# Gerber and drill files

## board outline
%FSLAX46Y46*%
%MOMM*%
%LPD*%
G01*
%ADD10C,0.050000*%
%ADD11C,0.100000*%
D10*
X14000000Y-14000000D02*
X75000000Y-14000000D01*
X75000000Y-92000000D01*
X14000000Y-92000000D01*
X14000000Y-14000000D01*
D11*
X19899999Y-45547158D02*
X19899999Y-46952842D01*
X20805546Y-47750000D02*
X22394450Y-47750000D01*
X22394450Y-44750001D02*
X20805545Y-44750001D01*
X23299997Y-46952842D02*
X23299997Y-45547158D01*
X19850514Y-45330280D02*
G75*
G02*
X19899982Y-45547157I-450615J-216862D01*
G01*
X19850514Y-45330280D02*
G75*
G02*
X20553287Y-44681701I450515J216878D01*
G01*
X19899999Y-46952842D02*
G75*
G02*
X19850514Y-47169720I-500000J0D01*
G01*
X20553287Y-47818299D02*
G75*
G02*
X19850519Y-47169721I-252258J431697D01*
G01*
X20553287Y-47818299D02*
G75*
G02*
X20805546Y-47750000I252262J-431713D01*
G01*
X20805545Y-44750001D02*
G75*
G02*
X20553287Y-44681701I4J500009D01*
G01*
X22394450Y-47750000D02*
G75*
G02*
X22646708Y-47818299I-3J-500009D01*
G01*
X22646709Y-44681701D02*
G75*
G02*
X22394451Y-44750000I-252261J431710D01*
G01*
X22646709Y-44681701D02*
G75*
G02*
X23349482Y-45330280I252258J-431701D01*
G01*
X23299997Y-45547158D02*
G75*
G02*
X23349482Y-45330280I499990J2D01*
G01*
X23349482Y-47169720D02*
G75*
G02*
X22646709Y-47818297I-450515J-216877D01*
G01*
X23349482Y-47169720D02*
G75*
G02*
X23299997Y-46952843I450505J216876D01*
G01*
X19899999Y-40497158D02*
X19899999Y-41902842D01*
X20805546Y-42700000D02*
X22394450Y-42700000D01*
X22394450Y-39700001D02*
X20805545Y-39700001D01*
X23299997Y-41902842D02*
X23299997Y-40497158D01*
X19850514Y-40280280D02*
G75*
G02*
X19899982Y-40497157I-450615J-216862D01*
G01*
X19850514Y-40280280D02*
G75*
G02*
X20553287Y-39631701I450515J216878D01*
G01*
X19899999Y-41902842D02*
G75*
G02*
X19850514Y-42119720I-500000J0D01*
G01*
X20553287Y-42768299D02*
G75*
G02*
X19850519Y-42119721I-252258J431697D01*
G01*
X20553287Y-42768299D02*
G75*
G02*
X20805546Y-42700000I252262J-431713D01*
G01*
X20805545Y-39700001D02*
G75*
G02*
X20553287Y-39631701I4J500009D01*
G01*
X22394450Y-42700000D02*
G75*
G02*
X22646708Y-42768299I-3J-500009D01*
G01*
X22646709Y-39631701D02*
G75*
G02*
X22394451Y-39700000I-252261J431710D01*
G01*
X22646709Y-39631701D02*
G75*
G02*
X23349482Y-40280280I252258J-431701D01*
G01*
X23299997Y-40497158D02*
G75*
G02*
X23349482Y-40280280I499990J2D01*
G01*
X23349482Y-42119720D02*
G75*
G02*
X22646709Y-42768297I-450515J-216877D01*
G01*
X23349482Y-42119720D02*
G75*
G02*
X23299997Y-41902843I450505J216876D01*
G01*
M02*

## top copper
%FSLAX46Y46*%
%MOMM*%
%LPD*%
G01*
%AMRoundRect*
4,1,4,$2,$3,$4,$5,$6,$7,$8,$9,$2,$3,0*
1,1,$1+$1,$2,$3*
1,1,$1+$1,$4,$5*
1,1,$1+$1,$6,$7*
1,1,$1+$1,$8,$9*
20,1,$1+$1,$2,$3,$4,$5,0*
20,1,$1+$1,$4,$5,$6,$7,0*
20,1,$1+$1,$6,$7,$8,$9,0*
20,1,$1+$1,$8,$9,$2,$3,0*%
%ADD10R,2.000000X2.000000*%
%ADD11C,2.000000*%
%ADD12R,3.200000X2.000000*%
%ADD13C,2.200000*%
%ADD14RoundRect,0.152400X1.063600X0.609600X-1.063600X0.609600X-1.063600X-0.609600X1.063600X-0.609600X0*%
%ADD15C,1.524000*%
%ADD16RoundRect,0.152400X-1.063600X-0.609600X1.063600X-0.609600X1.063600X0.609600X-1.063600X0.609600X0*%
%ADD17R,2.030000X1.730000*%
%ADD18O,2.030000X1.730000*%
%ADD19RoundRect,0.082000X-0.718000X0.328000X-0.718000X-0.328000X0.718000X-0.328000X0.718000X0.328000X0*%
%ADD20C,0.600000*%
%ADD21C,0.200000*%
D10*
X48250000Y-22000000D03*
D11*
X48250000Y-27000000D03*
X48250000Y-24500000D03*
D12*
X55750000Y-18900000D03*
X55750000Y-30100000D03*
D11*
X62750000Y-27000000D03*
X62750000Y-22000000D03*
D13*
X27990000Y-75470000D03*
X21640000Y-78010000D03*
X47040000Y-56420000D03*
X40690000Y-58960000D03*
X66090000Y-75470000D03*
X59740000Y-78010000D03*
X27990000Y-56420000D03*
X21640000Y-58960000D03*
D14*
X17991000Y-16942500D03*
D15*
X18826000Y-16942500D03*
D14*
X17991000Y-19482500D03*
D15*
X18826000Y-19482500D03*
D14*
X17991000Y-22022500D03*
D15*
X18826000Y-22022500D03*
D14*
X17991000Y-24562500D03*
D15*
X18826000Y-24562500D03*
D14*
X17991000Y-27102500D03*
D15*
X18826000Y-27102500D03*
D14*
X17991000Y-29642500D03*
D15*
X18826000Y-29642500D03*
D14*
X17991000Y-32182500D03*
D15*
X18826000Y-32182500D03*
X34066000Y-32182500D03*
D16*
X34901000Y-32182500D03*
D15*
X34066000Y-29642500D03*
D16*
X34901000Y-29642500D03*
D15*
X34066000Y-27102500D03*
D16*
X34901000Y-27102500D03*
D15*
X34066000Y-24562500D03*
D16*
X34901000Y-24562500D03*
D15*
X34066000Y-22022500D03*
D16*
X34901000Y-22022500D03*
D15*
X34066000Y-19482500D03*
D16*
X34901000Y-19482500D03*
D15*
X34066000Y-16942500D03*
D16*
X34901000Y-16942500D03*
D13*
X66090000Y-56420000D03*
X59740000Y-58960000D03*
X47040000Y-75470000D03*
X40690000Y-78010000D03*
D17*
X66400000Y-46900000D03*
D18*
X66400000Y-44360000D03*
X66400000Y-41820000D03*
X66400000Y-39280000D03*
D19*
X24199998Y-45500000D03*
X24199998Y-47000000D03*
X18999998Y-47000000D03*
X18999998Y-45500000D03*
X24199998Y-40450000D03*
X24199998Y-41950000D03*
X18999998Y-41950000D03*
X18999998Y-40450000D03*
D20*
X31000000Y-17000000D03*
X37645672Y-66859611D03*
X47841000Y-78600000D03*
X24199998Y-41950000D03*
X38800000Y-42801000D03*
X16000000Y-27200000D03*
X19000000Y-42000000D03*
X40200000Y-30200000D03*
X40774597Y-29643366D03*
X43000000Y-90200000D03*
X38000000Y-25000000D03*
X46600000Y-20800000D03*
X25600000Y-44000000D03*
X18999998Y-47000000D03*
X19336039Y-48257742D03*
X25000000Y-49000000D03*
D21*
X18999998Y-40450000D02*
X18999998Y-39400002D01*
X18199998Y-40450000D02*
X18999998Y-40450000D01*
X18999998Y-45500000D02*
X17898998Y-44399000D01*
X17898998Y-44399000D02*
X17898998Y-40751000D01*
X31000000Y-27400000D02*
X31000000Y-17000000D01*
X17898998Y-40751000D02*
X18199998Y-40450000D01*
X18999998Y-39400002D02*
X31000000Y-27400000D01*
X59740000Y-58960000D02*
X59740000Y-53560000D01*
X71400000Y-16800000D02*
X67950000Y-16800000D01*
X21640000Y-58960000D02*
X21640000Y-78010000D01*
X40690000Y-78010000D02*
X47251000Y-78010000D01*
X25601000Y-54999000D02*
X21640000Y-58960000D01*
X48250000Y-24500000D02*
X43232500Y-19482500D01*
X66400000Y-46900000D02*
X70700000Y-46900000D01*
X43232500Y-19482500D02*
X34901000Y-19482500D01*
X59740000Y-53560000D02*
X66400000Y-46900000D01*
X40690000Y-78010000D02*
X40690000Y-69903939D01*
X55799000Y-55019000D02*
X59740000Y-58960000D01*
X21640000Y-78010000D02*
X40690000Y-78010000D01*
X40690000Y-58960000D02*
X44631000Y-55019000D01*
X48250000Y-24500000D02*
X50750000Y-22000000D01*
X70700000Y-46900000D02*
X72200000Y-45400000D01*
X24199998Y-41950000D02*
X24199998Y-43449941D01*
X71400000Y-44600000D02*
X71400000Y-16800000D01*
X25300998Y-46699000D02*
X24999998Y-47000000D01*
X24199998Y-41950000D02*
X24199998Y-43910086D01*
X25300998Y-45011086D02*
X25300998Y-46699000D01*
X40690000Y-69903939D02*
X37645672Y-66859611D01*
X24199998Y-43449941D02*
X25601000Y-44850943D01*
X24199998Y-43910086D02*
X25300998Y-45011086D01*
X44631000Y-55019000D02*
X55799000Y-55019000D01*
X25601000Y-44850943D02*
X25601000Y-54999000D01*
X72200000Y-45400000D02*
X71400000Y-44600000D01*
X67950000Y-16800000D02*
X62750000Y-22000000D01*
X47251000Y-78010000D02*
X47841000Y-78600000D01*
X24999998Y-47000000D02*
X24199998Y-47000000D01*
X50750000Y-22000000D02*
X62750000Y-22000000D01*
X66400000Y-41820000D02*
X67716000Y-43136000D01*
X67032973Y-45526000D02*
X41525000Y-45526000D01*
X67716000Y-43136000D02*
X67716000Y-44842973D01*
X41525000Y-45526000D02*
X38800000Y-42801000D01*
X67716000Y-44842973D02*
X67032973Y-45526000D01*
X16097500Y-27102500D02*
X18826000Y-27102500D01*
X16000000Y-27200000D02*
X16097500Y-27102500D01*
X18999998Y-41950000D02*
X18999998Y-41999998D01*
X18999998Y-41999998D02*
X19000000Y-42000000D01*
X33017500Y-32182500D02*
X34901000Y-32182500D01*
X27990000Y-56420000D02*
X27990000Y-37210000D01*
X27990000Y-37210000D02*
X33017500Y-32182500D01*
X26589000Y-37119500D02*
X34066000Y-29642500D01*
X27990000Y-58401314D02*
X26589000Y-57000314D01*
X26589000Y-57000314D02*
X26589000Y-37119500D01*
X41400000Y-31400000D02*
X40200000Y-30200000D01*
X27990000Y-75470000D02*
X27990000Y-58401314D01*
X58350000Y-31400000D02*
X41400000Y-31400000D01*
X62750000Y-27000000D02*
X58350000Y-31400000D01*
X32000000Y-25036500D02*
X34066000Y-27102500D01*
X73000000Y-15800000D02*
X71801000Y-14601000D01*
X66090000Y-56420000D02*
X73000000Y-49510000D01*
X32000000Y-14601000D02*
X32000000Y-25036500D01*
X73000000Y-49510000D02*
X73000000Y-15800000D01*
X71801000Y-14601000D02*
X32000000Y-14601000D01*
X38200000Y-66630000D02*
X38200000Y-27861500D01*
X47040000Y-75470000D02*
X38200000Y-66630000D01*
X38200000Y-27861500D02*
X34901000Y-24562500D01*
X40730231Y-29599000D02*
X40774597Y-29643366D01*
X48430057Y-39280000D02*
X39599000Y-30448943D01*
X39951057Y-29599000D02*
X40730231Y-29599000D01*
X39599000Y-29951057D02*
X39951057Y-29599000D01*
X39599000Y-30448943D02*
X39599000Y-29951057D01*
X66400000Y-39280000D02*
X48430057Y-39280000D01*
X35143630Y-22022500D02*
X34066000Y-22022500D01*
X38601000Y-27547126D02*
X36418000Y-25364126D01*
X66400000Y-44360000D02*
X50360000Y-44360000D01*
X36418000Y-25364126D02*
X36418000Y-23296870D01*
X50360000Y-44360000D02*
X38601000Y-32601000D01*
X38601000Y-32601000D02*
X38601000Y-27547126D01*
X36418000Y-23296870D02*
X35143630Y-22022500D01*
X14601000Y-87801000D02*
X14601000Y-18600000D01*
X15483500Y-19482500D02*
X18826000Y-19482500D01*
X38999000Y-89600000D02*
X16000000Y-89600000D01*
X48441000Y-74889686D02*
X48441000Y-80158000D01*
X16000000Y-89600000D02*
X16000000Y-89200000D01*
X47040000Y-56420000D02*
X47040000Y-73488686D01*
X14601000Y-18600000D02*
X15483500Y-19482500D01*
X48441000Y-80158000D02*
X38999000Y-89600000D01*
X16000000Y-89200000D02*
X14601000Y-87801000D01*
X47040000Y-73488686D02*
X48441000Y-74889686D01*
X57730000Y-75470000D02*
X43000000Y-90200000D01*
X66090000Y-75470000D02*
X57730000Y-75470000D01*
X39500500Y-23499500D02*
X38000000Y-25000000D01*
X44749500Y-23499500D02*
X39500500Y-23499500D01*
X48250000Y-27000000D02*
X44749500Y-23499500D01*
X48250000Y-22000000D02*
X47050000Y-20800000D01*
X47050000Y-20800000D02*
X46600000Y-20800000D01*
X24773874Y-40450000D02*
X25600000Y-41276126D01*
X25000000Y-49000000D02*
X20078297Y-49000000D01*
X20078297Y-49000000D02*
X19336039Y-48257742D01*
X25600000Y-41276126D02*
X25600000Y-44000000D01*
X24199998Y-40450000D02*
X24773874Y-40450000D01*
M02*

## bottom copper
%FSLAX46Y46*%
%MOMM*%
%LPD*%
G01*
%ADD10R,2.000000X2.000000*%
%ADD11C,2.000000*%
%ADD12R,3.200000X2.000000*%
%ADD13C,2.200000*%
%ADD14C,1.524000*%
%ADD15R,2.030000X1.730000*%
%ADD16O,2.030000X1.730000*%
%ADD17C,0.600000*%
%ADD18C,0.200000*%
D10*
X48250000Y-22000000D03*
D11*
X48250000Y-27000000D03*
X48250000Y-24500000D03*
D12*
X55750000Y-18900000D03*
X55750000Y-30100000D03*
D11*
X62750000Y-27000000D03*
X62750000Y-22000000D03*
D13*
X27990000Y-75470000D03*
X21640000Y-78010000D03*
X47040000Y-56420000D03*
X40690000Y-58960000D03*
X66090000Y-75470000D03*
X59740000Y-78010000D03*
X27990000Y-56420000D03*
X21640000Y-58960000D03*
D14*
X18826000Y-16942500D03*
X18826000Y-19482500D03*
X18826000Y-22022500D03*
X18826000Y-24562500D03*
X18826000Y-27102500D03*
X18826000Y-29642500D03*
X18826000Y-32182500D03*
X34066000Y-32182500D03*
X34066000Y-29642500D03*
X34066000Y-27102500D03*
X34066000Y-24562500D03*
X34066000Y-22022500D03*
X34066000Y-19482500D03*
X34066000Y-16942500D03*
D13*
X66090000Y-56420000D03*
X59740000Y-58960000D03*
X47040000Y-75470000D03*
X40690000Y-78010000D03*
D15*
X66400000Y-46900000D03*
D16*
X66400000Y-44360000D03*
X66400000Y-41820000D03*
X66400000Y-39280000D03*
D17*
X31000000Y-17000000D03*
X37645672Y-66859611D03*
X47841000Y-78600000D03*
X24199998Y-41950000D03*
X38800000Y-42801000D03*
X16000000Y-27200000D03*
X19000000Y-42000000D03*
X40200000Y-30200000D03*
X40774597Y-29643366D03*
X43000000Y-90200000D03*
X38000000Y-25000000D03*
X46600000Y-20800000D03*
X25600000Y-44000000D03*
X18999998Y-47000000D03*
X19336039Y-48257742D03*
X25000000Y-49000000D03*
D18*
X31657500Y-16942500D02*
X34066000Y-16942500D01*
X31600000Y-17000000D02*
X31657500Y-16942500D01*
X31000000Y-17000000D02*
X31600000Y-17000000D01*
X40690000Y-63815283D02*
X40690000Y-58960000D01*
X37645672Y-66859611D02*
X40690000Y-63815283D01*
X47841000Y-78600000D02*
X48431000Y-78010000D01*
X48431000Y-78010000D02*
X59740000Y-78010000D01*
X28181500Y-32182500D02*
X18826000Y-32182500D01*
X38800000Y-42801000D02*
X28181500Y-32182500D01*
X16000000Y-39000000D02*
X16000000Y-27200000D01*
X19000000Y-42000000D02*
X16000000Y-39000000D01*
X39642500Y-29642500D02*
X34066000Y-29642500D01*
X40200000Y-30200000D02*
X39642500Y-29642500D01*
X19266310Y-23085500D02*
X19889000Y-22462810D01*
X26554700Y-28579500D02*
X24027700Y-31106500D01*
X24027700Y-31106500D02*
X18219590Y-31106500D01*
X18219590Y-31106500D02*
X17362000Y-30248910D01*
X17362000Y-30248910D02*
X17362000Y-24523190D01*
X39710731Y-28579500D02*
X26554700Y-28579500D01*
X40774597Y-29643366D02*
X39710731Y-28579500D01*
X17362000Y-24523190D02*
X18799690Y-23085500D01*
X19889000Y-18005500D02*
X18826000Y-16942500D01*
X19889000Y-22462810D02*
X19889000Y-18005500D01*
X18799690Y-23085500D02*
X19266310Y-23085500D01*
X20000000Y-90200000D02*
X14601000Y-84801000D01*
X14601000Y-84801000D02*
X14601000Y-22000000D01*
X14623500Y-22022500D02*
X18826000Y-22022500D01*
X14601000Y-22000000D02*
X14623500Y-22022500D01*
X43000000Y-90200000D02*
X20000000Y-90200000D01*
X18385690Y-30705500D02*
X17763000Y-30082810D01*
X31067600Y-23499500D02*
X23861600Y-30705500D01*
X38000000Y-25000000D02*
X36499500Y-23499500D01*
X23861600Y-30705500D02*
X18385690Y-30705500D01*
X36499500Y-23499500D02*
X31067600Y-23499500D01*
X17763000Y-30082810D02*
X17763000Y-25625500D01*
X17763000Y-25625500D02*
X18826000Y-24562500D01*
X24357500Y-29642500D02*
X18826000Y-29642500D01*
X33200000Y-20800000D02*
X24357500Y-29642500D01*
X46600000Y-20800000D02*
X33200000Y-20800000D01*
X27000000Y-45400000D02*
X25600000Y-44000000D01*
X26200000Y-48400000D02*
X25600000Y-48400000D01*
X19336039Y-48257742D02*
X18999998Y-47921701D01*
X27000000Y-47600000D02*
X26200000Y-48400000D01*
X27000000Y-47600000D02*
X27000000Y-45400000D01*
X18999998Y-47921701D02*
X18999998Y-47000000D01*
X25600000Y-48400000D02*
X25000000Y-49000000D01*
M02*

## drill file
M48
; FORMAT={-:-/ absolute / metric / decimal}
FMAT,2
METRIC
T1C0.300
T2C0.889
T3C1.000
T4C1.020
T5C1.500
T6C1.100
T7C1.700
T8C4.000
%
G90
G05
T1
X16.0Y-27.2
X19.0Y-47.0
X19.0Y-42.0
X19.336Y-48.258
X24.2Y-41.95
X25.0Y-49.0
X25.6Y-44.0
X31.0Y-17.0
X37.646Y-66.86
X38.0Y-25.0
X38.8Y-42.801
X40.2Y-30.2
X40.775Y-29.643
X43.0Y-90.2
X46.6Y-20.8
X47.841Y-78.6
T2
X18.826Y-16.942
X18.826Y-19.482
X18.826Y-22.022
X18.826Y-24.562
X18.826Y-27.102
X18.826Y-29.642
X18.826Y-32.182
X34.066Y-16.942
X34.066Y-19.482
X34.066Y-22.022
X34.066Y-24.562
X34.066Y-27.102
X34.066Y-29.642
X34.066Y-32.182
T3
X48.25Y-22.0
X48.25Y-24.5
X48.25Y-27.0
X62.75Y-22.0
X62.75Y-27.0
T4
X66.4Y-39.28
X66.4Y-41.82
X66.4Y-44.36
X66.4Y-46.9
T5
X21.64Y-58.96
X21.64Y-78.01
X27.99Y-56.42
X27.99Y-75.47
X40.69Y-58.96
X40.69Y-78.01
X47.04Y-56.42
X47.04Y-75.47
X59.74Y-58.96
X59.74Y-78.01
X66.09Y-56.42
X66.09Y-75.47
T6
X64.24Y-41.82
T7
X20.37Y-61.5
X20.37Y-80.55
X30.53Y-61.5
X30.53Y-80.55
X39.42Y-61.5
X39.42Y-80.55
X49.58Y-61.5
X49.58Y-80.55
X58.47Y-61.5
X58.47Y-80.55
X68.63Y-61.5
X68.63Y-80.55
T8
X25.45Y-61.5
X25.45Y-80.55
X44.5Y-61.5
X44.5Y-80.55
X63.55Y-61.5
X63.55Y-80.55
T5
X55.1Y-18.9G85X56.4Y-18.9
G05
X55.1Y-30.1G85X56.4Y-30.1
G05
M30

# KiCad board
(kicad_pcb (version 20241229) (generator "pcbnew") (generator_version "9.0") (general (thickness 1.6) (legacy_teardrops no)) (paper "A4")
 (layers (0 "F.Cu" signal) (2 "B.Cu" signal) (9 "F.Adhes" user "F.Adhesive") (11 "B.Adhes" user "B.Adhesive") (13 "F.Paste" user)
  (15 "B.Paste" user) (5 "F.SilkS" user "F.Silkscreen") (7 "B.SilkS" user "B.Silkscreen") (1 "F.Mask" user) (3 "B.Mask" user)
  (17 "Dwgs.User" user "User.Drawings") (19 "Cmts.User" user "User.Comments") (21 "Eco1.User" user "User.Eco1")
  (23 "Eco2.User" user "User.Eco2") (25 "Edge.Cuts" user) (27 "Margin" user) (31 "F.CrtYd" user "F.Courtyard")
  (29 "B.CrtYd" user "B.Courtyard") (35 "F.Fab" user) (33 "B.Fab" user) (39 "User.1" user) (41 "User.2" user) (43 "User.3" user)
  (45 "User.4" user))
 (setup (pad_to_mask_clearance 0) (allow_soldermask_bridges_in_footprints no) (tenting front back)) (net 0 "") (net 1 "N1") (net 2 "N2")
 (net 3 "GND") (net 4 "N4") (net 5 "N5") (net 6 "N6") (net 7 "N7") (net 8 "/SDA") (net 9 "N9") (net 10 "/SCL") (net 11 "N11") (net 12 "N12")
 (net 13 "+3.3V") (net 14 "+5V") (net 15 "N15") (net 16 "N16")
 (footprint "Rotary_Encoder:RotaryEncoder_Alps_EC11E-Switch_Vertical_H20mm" (layer "F.Cu") (at 48.25 22)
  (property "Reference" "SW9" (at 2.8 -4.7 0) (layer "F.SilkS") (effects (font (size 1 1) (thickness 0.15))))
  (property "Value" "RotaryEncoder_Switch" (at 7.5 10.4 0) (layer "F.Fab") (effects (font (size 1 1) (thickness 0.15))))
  (pad "A" thru_hole rect (at 0 0) (size 2 2) (drill 1) (layers "*.Cu" "*.Mask") (remove_unused_layers no) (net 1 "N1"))
  (pad "B" thru_hole circle (at 0 5) (size 2 2) (drill 1) (layers "*.Cu" "*.Mask") (remove_unused_layers no) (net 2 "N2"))
  (pad "C" thru_hole circle (at 0 2.5) (size 2 2) (drill 1) (layers "*.Cu" "*.Mask") (remove_unused_layers no) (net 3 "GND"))
  (pad "MP" thru_hole rect (at 7.5 -3.1) (size 3.2 2) (drill oval 2.8 1.5) (layers "*.Cu" "*.Mask") (remove_unused_layers no))
  (pad "MP" thru_hole rect (at 7.5 8.1) (size 3.2 2) (drill oval 2.8 1.5) (layers "*.Cu" "*.Mask") (remove_unused_layers no))
  (pad "S1" thru_hole circle (at 14.5 5) (size 2 2) (drill 1) (layers "*.Cu" "*.Mask") (remove_unused_layers no) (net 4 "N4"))
  (pad "S2" thru_hole circle (at 14.5 0) (size 2 2) (drill 1) (layers "*.Cu" "*.Mask") (remove_unused_layers no) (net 3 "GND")))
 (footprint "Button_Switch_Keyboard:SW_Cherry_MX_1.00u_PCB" (layer "F.Cu") (at 27.99 75.47)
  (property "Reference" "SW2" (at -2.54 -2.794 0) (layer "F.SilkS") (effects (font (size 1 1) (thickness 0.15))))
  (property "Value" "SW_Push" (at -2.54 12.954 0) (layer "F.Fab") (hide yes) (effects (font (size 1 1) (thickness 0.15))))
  (pad "" np_thru_hole circle (at -7.62 5.08) (size 1.7 1.7) (drill 1.7) (layers "*.Cu" "*.Mask"))
  (pad "" np_thru_hole circle (at -2.54 5.08) (size 4 4) (drill 4) (layers "*.Cu" "*.Mask"))
  (pad "" np_thru_hole circle (at 2.54 5.08) (size 1.7 1.7) (drill 1.7) (layers "*.Cu" "*.Mask"))
  (pad "1" thru_hole circle (at 0 0) (size 2.2 2.2) (drill 1.5) (layers "*.Cu" "*.Mask") (remove_unused_layers no) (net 4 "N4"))
  (pad "2" thru_hole circle (at -6.35 2.54) (size 2.2 2.2) (drill 1.5) (layers "*.Cu" "*.Mask") (remove_unused_layers no) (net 3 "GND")))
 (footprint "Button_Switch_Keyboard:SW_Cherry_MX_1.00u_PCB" (layer "F.Cu") (at 47.04 56.42)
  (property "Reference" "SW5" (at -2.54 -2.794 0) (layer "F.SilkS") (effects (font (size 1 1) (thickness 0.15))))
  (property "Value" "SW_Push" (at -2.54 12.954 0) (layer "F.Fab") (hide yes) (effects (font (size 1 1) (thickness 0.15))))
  (pad "" np_thru_hole circle (at -7.62 5.08) (size 1.7 1.7) (drill 1.7) (layers "*.Cu" "*.Mask"))
  (pad "" np_thru_hole circle (at -2.54 5.08) (size 4 4) (drill 4) (layers "*.Cu" "*.Mask"))
  (pad "" np_thru_hole circle (at 2.54 5.08) (size 1.7 1.7) (drill 1.7) (layers "*.Cu" "*.Mask"))
  (pad "1" thru_hole circle (at 0 0) (size 2.2 2.2) (drill 1.5) (layers "*.Cu" "*.Mask") (remove_unused_layers no) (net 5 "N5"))
  (pad "2" thru_hole circle (at -6.35 2.54) (size 2.2 2.2) (drill 1.5) (layers "*.Cu" "*.Mask") (remove_unused_layers no) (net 3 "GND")))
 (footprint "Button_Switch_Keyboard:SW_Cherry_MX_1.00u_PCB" (layer "F.Cu") (at 66.09 75.47)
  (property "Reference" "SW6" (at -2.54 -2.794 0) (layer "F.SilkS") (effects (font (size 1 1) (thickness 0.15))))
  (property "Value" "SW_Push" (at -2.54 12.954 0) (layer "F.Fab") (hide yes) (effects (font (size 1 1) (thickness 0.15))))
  (pad "" np_thru_hole circle (at -7.62 5.08) (size 1.7 1.7) (drill 1.7) (layers "*.Cu" "*.Mask"))
  (pad "" np_thru_hole circle (at -2.54 5.08) (size 4 4) (drill 4) (layers "*.Cu" "*.Mask"))
  (pad "" np_thru_hole circle (at 2.54 5.08) (size 1.7 1.7) (drill 1.7) (layers "*.Cu" "*.Mask"))
  (pad "1" thru_hole circle (at 0 0) (size 2.2 2.2) (drill 1.5) (layers "*.Cu" "*.Mask") (remove_unused_layers no) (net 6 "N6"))
  (pad "2" thru_hole circle (at -6.35 2.54) (size 2.2 2.2) (drill 1.5) (layers "*.Cu" "*.Mask") (remove_unused_layers no) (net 3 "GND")))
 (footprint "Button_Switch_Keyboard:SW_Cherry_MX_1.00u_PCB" (layer "F.Cu") (at 27.99 56.42)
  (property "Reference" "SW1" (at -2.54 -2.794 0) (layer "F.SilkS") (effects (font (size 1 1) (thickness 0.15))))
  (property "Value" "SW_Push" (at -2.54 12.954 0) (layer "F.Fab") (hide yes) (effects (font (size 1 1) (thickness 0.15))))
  (pad "" np_thru_hole circle (at -7.62 5.08) (size 1.7 1.7) (drill 1.7) (layers "*.Cu" "*.Mask"))
  (pad "" np_thru_hole circle (at -2.54 5.08) (size 4 4) (drill 4) (layers "*.Cu" "*.Mask"))
  (pad "" np_thru_hole circle (at 2.54 5.08) (size 1.7 1.7) (drill 1.7) (layers "*.Cu" "*.Mask"))
  (pad "1" thru_hole circle (at 0 0) (size 2.2 2.2) (drill 1.5) (layers "*.Cu" "*.Mask") (remove_unused_layers no) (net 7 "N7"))
  (pad "2" thru_hole circle (at -6.35 2.54) (size 2.2 2.2) (drill 1.5) (layers "*.Cu" "*.Mask") (remove_unused_layers no) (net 3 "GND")))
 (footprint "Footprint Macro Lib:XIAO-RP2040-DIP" (layer "F.Cu") (at 26.446 24.5625)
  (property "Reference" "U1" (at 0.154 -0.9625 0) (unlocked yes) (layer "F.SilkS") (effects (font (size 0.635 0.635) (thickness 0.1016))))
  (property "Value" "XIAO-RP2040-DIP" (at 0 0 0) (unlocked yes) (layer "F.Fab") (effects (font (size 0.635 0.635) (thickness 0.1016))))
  (pad "1" smd roundrect (at -8.455 -7.62 180) (size 2.432 1.524) (layers "F.Cu" "F.Mask") (roundrect_rratio 0.1) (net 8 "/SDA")
   (thermal_bridge_angle 45))
  (pad "1" thru_hole circle (at -7.62 -7.62 180) (size 1.524 1.524) (drill 0.889) (layers "*.Cu" "*.Mask") (remove_unused_layers no)
   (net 8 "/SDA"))
  (pad "2" smd roundrect (at -8.455 -5.08 180) (size 2.432 1.524) (layers "F.Cu" "F.Mask") (roundrect_rratio 0.1) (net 5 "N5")
   (thermal_bridge_angle 45))
  (pad "2" thru_hole circle (at -7.62 -5.08 180) (size 1.524 1.524) (drill 0.889) (layers "*.Cu" "*.Mask") (remove_unused_layers no)
   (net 5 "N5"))
  (pad "3" smd roundrect (at -8.455 -2.54 180) (size 2.432 1.524) (layers "F.Cu" "F.Mask") (roundrect_rratio 0.1) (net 6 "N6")
   (thermal_bridge_angle 45))
  (pad "3" thru_hole circle (at -7.62 -2.54 180) (size 1.524 1.524) (drill 0.889) (layers "*.Cu" "*.Mask") (remove_unused_layers no)
   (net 6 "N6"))
  (pad "4" smd roundrect (at -8.455 0 180) (size 2.432 1.524) (layers "F.Cu" "F.Mask") (roundrect_rratio 0.1) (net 2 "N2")
   (thermal_bridge_angle 45))
  (pad "4" thru_hole circle (at -7.62 0 180) (size 1.524 1.524) (drill 0.889) (layers "*.Cu" "*.Mask") (remove_unused_layers no)
   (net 2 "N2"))
  (pad "5" smd roundrect (at -8.455 2.54 180) (size 2.432 1.524) (layers "F.Cu" "F.Mask") (roundrect_rratio 0.1) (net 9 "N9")
   (thermal_bridge_angle 45))
  (pad "5" thru_hole circle (at -7.62 2.54 180) (size 1.524 1.524) (drill 0.889) (layers "*.Cu" "*.Mask") (remove_unused_layers no)
   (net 9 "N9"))
  (pad "6" smd roundrect (at -8.455 5.08 180) (size 2.432 1.524) (layers "F.Cu" "F.Mask") (roundrect_rratio 0.1) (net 1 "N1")
   (thermal_bridge_angle 45))
  (pad "6" thru_hole circle (at -7.62 5.08 180) (size 1.524 1.524) (drill 0.889) (layers "*.Cu" "*.Mask") (remove_unused_layers no)
   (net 1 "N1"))
  (pad "7" smd roundrect (at -8.455 7.62 180) (size 2.432 1.524) (layers "F.Cu" "F.Mask") (roundrect_rratio 0.1) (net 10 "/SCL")
   (thermal_bridge_angle 45))
  (pad "7" thru_hole circle (at -7.62 7.62 180) (size 1.524 1.524) (drill 0.889) (layers "*.Cu" "*.Mask") (remove_unused_layers no)
   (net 10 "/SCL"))
  (pad "8" thru_hole circle (at 7.62 7.62) (size 1.524 1.524) (drill 0.889) (layers "*.Cu" "*.Mask") (remove_unused_layers no) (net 7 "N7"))
  (pad "8" smd roundrect (at 8.455 7.62) (size 2.432 1.524) (layers "F.Cu" "F.Mask") (roundrect_rratio 0.1) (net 7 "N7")
   (thermal_bridge_angle 45))
  (pad "9" thru_hole circle (at 7.62 5.08) (size 1.524 1.524) (drill 0.889) (layers "*.Cu" "*.Mask") (remove_unused_layers no) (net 4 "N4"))
  (pad "9" smd roundrect (at 8.455 5.08) (size 2.432 1.524) (layers "F.Cu" "F.Mask") (roundrect_rratio 0.1) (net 4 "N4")
   (thermal_bridge_angle 45))
  (pad "10" thru_hole circle (at 7.62 2.54) (size 1.524 1.524) (drill 0.889) (layers "*.Cu" "*.Mask") (remove_unused_layers no)
   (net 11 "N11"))
  (pad "10" smd roundrect (at 8.455 2.54) (size 2.432 1.524) (layers "F.Cu" "F.Mask") (roundrect_rratio 0.1) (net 11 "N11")
   (thermal_bridge_angle 45))
  (pad "11" thru_hole circle (at 7.62 0) (size 1.524 1.524) (drill 0.889) (layers "*.Cu" "*.Mask") (remove_unused_layers no) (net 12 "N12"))
  (pad "11" smd roundrect (at 8.455 0) (size 2.432 1.524) (layers "F.Cu" "F.Mask") (roundrect_rratio 0.1) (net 12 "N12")
   (thermal_bridge_angle 45))
  (pad "12" thru_hole circle (at 7.62 -2.54) (size 1.524 1.524) (drill 0.889) (layers "*.Cu" "*.Mask") (remove_unused_layers no)
   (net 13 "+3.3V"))
  (pad "12" smd roundrect (at 8.455 -2.54) (size 2.432 1.524) (layers "F.Cu" "F.Mask") (roundrect_rratio 0.1) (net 13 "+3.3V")
   (thermal_bridge_angle 45))
  (pad "13" thru_hole circle (at 7.62 -5.08) (size 1.524 1.524) (drill 0.889) (layers "*.Cu" "*.Mask") (remove_unused_layers no)
   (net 3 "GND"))
  (pad "13" smd roundrect (at 8.455 -5.08) (size 2.432 1.524) (layers "F.Cu" "F.Mask") (roundrect_rratio 0.1) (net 3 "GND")
   (thermal_bridge_angle 45))
  (pad "14" thru_hole circle (at 7.62 -7.62) (size 1.524 1.524) (drill 0.889) (layers "*.Cu" "*.Mask") (remove_unused_layers no)
   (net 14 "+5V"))
  (pad "14" smd roundrect (at 8.455 -7.62) (size 2.432 1.524) (layers "F.Cu" "F.Mask") (roundrect_rratio 0.1) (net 14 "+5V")
   (thermal_bridge_angle 45)))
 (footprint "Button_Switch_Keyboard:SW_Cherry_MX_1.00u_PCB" (layer "F.Cu") (at 66.09 56.42)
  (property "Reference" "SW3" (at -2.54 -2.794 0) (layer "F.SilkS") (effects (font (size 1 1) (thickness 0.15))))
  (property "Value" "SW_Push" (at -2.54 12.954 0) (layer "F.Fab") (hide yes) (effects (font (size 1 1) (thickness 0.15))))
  (pad "" np_thru_hole circle (at -7.62 5.08) (size 1.7 1.7) (drill 1.7) (layers "*.Cu" "*.Mask"))
  (pad "" np_thru_hole circle (at -2.54 5.08) (size 4 4) (drill 4) (layers "*.Cu" "*.Mask"))
  (pad "" np_thru_hole circle (at 2.54 5.08) (size 1.7 1.7) (drill 1.7) (layers "*.Cu" "*.Mask"))
  (pad "1" thru_hole circle (at 0 0) (size 2.2 2.2) (drill 1.5) (layers "*.Cu" "*.Mask") (remove_unused_layers no) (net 11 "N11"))
  (pad "2" thru_hole circle (at -6.35 2.54) (size 2.2 2.2) (drill 1.5) (layers "*.Cu" "*.Mask") (remove_unused_layers no) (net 3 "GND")))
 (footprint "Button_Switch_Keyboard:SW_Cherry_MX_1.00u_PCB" (layer "F.Cu") (at 47.04 75.47)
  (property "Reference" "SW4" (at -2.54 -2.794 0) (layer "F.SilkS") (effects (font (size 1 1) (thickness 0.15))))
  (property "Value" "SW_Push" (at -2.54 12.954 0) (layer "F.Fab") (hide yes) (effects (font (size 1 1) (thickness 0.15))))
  (pad "" np_thru_hole circle (at -7.62 5.08) (size 1.7 1.7) (drill 1.7) (layers "*.Cu" "*.Mask"))
  (pad "" np_thru_hole circle (at -2.54 5.08) (size 4 4) (drill 4) (layers "*.Cu" "*.Mask"))
  (pad "" np_thru_hole circle (at 2.54 5.08) (size 1.7 1.7) (drill 1.7) (layers "*.Cu" "*.Mask"))
  (pad "1" thru_hole circle (at 0 0) (size 2.2 2.2) (drill 1.5) (layers "*.Cu" "*.Mask") (remove_unused_layers no) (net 12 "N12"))
  (pad "2" thru_hole circle (at -6.35 2.54) (size 2.2 2.2) (drill 1.5) (layers "*.Cu" "*.Mask") (remove_unused_layers no) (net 3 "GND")))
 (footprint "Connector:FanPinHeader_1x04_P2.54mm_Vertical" (layer "F.Cu") (at 66.4 46.9 90)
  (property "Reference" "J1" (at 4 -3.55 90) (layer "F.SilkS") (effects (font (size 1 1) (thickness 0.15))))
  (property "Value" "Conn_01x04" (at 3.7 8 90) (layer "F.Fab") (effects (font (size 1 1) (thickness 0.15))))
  (pad "" np_thru_hole circle (at 5.08 -2.16 180) (size 1.1 1.1) (drill 1.1) (layers "*.Cu" "*.Mask"))
  (pad "1" thru_hole rect (at 0 0 180) (size 2.03 1.73) (drill 1.02) (layers "*.Cu" "*.Mask") (remove_unused_layers no) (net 3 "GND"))
  (pad "2" thru_hole oval (at 2.54 0 180) (size 2.03 1.73) (drill 1.02) (layers "*.Cu" "*.Mask") (remove_unused_layers no) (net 13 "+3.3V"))
  (pad "3" thru_hole oval (at 5.08 0 180) (size 2.03 1.73) (drill 1.02) (layers "*.Cu" "*.Mask") (remove_unused_layers no) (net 10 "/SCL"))
  (pad "4" thru_hole oval (at 7.62 0 180) (size 2.03 1.73) (drill 1.02) (layers "*.Cu" "*.Mask") (remove_unused_layers no) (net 8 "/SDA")))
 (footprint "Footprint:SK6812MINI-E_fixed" (layer "B.Cu") (at 21.599999 46.352842 180)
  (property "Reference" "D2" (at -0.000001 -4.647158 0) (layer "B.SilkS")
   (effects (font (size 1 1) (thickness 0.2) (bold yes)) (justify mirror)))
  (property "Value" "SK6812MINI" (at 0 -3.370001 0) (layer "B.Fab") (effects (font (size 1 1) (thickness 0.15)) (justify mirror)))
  (fp_line (start 1.7 0.805684) (end 1.7 -0.6) (stroke (width 0.1) (type solid)) (layer "Edge.Cuts"))
  (fp_line (start 0.794453 -1.397158) (end -0.794451 -1.397158) (stroke (width 0.1) (type solid)) (layer "Edge.Cuts"))
  (fp_line (start -0.794451 1.602841) (end 0.794454 1.602841) (stroke (width 0.1) (type solid)) (layer "Edge.Cuts"))
  (fp_line (start -1.699998 -0.6) (end -1.699998 0.805684) (stroke (width 0.1) (type solid)) (layer "Edge.Cuts"))
  (fp_arc (start 1.749485 1.022562) (mid 1.712532 0.91691) (end 1.7 0.805685) (stroke (width 0.1) (type solid)) (layer "Edge.Cuts"))
  (fp_arc (start 1.749485 1.022562) (mid 1.638072 1.606877) (end 1.046712 1.67114) (stroke (width 0.1) (type solid)) (layer "Edge.Cuts"))
  (fp_arc (start 1.7 -0.6) (mid 1.712528 -0.711226) (end 1.749485 -0.816878) (stroke (width 0.1) (type solid)) (layer "Edge.Cuts"))
  (fp_arc (start 1.046712 -1.465457) (mid 1.638073 -1.401193) (end 1.749485 -0.816877) (stroke (width 0.1) (type solid)) (layer "Edge.Cuts"))
  (fp_arc (start 1.046712 -1.465457) (mid 0.925124 -1.414535) (end 0.794453 -1.397158) (stroke (width 0.1) (type solid)) (layer "Edge.Cuts"))
  (fp_arc (start 0.794454 1.602841) (mid 0.925124 1.620218) (end 1.046712 1.67114) (stroke (width 0.1) (type solid)) (layer "Edge.Cuts"))
  (fp_arc (start -0.794451 -1.397158) (mid -0.925121 -1.414535) (end -1.046709 -1.465457) (stroke (width 0.1) (type solid))
   (layer "Edge.Cuts"))
  (fp_arc (start -1.04671 1.671141) (mid -0.925122 1.620219) (end -0.794452 1.602842) (stroke (width 0.1) (type solid)) (layer "Edge.Cuts"))
  (fp_arc (start -1.04671 1.671141) (mid -1.63807 1.606877) (end -1.749483 1.022562) (stroke (width 0.1) (type solid)) (layer "Edge.Cuts"))
  (fp_arc (start -1.699998 0.805684) (mid -1.712526 0.91691) (end -1.749483 1.022562) (stroke (width 0.1) (type solid)) (layer "Edge.Cuts"))
  (fp_arc (start -1.749483 -0.816878) (mid -1.638069 -1.401192) (end -1.04671 -1.465455) (stroke (width 0.1) (type solid))
   (layer "Edge.Cuts"))
  (fp_arc (start -1.749483 -0.816878) (mid -1.712526 -0.711226) (end -1.699998 -0.600001) (stroke (width 0.1) (type solid))
   (layer "Edge.Cuts"))
  (pad "1" smd roundrect (at -2.599999 0.852842 270) (size 0.82 1.6) (layers "F.Cu" "F.Mask" "F.Paste") (roundrect_rratio 0.1)
   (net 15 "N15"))
  (pad "2" smd roundrect (at -2.599999 -0.647158 270) (size 0.82 1.6) (layers "F.Cu" "F.Mask" "F.Paste") (roundrect_rratio 0.1)
   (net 3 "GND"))
  (pad "3" smd roundrect (at 2.600001 -0.647158 270) (size 0.82 1.6) (layers "F.Cu" "F.Mask" "F.Paste") (roundrect_rratio 0.1)
   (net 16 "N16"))
  (pad "4" smd roundrect (at 2.600001 0.852842 270) (size 0.82 1.6) (layers "F.Cu" "F.Mask" "F.Paste") (roundrect_rratio 0.1) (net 14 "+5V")))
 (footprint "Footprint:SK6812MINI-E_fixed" (layer "B.Cu") (at 21.599999 41.302842 180)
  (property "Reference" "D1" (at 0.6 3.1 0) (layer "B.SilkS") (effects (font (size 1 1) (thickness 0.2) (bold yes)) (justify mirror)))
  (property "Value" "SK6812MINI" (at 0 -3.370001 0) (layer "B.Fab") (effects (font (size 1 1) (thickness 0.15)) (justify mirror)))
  (fp_line (start 1.7 0.805684) (end 1.7 -0.6) (stroke (width 0.1) (type solid)) (layer "Edge.Cuts"))
  (fp_line (start 0.794453 -1.397158) (end -0.794451 -1.397158) (stroke (width 0.1) (type solid)) (layer "Edge.Cuts"))
  (fp_line (start -0.794451 1.602841) (end 0.794454 1.602841) (stroke (width 0.1) (type solid)) (layer "Edge.Cuts"))
  (fp_line (start -1.699998 -0.6) (end -1.699998 0.805684) (stroke (width 0.1) (type solid)) (layer "Edge.Cuts"))
  (fp_arc (start 1.749485 1.022562) (mid 1.712532 0.91691) (end 1.7 0.805685) (stroke (width 0.1) (type solid)) (layer "Edge.Cuts"))
  (fp_arc (start 1.749485 1.022562) (mid 1.638072 1.606877) (end 1.046712 1.67114) (stroke (width 0.1) (type solid)) (layer "Edge.Cuts"))
  (fp_arc (start 1.7 -0.6) (mid 1.712528 -0.711226) (end 1.749485 -0.816878) (stroke (width 0.1) (type solid)) (layer "Edge.Cuts"))
  (fp_arc (start 1.046712 -1.465457) (mid 1.638073 -1.401193) (end 1.749485 -0.816877) (stroke (width 0.1) (type solid)) (layer "Edge.Cuts"))
  (fp_arc (start 1.046712 -1.465457) (mid 0.925124 -1.414535) (end 0.794453 -1.397158) (stroke (width 0.1) (type solid)) (layer "Edge.Cuts"))
  (fp_arc (start 0.794454 1.602841) (mid 0.925124 1.620218) (end 1.046712 1.67114) (stroke (width 0.1) (type solid)) (layer "Edge.Cuts"))
  (fp_arc (start -0.794451 -1.397158) (mid -0.925121 -1.414535) (end -1.046709 -1.465457) (stroke (width 0.1) (type solid))
   (layer "Edge.Cuts"))
  (fp_arc (start -1.04671 1.671141) (mid -0.925122 1.620219) (end -0.794452 1.602842) (stroke (width 0.1) (type solid)) (layer "Edge.Cuts"))
  (fp_arc (start -1.04671 1.671141) (mid -1.63807 1.606877) (end -1.749483 1.022562) (stroke (width 0.1) (type solid)) (layer "Edge.Cuts"))
  (fp_arc (start -1.699998 0.805684) (mid -1.712526 0.91691) (end -1.749483 1.022562) (stroke (width 0.1) (type solid)) (layer "Edge.Cuts"))
  (fp_arc (start -1.749483 -0.816878) (mid -1.638069 -1.401192) (end -1.04671 -1.465455) (stroke (width 0.1) (type solid))
   (layer "Edge.Cuts"))
  (fp_arc (start -1.749483 -0.816878) (mid -1.712526 -0.711226) (end -1.699998 -0.600001) (stroke (width 0.1) (type solid))
   (layer "Edge.Cuts"))
  (pad "1" smd roundrect (at -2.599999 0.852842 270) (size 0.82 1.6) (layers "F.Cu" "F.Mask" "F.Paste") (roundrect_rratio 0.1)
   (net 16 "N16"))
  (pad "2" smd roundrect (at -2.599999 -0.647158 270) (size 0.82 1.6) (layers "F.Cu" "F.Mask" "F.Paste") (roundrect_rratio 0.1)
   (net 3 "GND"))
  (pad "3" smd roundrect (at 2.600001 -0.647158 270) (size 0.82 1.6) (layers "F.Cu" "F.Mask" "F.Paste") (roundrect_rratio 0.1) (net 9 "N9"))
  (pad "4" smd roundrect (at 2.600001 0.852842 270) (size 0.82 1.6) (layers "F.Cu" "F.Mask" "F.Paste") (roundrect_rratio 0.1) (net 14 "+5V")))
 (gr_rect (start 14 14) (end 75 92) (stroke (width 0.05) (type solid)) (fill no) (layer "Edge.Cuts"))
 (segment (start 18.999998 40.45) (end 18.999998 39.400002) (width 0.2) (layer "F.Cu") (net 14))
 (segment (start 18.199998 40.45) (end 18.999998 40.45) (width 0.2) (layer "F.Cu") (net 14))
 (segment (start 18.999998 45.5) (end 17.898998 44.399) (width 0.2) (layer "F.Cu") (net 14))
 (segment (start 17.898998 44.399) (end 17.898998 40.751) (width 0.2) (layer "F.Cu") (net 14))
 (segment (start 31 27.4) (end 31 17) (width 0.2) (layer "F.Cu") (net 14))
 (segment (start 17.898998 40.751) (end 18.199998 40.45) (width 0.2) (layer "F.Cu") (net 14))
 (segment (start 18.999998 39.400002) (end 31 27.4) (width 0.2) (layer "F.Cu") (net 14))
 (via (at 31 17) (size 0.6) (drill 0.3) (layers "F.Cu" "B.Cu") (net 14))
 (segment (start 31.6575 16.9425) (end 34.066 16.9425) (width 0.2) (layer "B.Cu") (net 14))
 (segment (start 31.6 17) (end 31.6575 16.9425) (width 0.2) (layer "B.Cu") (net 14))
 (segment (start 31 17) (end 31.6 17) (width 0.2) (layer "B.Cu") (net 14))
 (segment (start 59.74 58.96) (end 59.74 53.56) (width 0.2) (layer "F.Cu") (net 3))
 (segment (start 71.4 16.8) (end 67.95 16.8) (width 0.2) (layer "F.Cu") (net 3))
 (segment (start 21.64 58.96) (end 21.64 78.01) (width 0.2) (layer "F.Cu") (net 3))
 (segment (start 40.69 78.01) (end 47.251 78.01) (width 0.2) (layer "F.Cu") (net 3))
 (segment (start 25.601 54.999) (end 21.64 58.96) (width 0.2) (layer "F.Cu") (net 3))
 (segment (start 48.25 24.5) (end 43.2325 19.4825) (width 0.2) (layer "F.Cu") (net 3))
 (segment (start 66.4 46.9) (end 70.7 46.9) (width 0.2) (layer "F.Cu") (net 3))
 (segment (start 43.2325 19.4825) (end 34.901 19.4825) (width 0.2) (layer "F.Cu") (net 3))
 (segment (start 59.74 53.56) (end 66.4 46.9) (width 0.2) (layer "F.Cu") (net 3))
 (segment (start 40.69 78.01) (end 40.69 69.903939) (width 0.2) (layer "F.Cu") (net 3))
 (segment (start 55.799 55.019) (end 59.74 58.96) (width 0.2) (layer "F.Cu") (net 3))
 (segment (start 21.64 78.01) (end 40.69 78.01) (width 0.2) (layer "F.Cu") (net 3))
 (segment (start 40.69 58.96) (end 44.631 55.019) (width 0.2) (layer "F.Cu") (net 3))
 (segment (start 48.25 24.5) (end 50.75 22) (width 0.2) (layer "F.Cu") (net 3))
 (segment (start 70.7 46.9) (end 72.2 45.4) (width 0.2) (layer "F.Cu") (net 3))
 (segment (start 24.199998 41.95) (end 24.199998 43.449941) (width 0.2) (layer "F.Cu") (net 3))
 (segment (start 71.4 44.6) (end 71.4 16.8) (width 0.2) (layer "F.Cu") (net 3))
 (segment (start 25.300998 46.699) (end 24.999998 47) (width 0.2) (layer "F.Cu") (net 3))
 (segment (start 24.199998 41.95) (end 24.199998 43.910086) (width 0.2) (layer "F.Cu") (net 3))
 (segment (start 25.300998 45.011086) (end 25.300998 46.699) (width 0.2) (layer "F.Cu") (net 3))
 (segment (start 40.69 69.903939) (end 37.645672 66.859611) (width 0.2) (layer "F.Cu") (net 3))
 (segment (start 24.199998 43.449941) (end 25.601 44.850943) (width 0.2) (layer "F.Cu") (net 3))
 (segment (start 24.199998 43.910086) (end 25.300998 45.011086) (width 0.2) (layer "F.Cu") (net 3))
 (segment (start 44.631 55.019) (end 55.799 55.019) (width 0.2) (layer "F.Cu") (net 3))
 (segment (start 25.601 44.850943) (end 25.601 54.999) (width 0.2) (layer "F.Cu") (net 3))
 (segment (start 72.2 45.4) (end 71.4 44.6) (width 0.2) (layer "F.Cu") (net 3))
 (segment (start 67.95 16.8) (end 62.75 22) (width 0.2) (layer "F.Cu") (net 3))
 (segment (start 47.251 78.01) (end 47.841 78.6) (width 0.2) (layer "F.Cu") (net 3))
 (segment (start 24.999998 47) (end 24.199998 47) (width 0.2) (layer "F.Cu") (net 3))
 (segment (start 50.75 22) (end 62.75 22) (width 0.2) (layer "F.Cu") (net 3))
 (via (at 37.645672 66.859611) (size 0.6) (drill 0.3) (layers "F.Cu" "B.Cu") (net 3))
 (via (at 47.841 78.6) (size 0.6) (drill 0.3) (layers "F.Cu" "B.Cu") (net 3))
 (via (at 24.199998 41.95) (size 0.6) (drill 0.3) (layers "F.Cu" "B.Cu") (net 3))
 (segment (start 40.69 63.815283) (end 40.69 58.96) (width 0.2) (layer "B.Cu") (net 3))
 (segment (start 37.645672 66.859611) (end 40.69 63.815283) (width 0.2) (layer "B.Cu") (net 3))
 (segment (start 47.841 78.6) (end 48.431 78.01) (width 0.2) (layer "B.Cu") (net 3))
 (segment (start 48.431 78.01) (end 59.74 78.01) (width 0.2) (layer "B.Cu") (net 3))
 (segment (start 66.4 41.82) (end 67.716 43.136) (width 0.2) (layer "F.Cu") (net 10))
 (segment (start 67.032973 45.526) (end 41.525 45.526) (width 0.2) (layer "F.Cu") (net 10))
 (segment (start 67.716 43.136) (end 67.716 44.842973) (width 0.2) (layer "F.Cu") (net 10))
 (segment (start 41.525 45.526) (end 38.8 42.801) (width 0.2) (layer "F.Cu") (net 10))
 (segment (start 67.716 44.842973) (end 67.032973 45.526) (width 0.2) (layer "F.Cu") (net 10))
 (via (at 38.8 42.801) (size 0.6) (drill 0.3) (layers "F.Cu" "B.Cu") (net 10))
 (segment (start 28.1815 32.1825) (end 18.826 32.1825) (width 0.2) (layer "B.Cu") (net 10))
 (segment (start 38.8 42.801) (end 28.1815 32.1825) (width 0.2) (layer "B.Cu") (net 10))
 (segment (start 16.0975 27.1025) (end 18.826 27.1025) (width 0.2) (layer "F.Cu") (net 9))
 (segment (start 16 27.2) (end 16.0975 27.1025) (width 0.2) (layer "F.Cu") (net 9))
 (segment (start 18.999998 41.95) (end 18.999998 41.999998) (width 0.2) (layer "F.Cu") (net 9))
 (segment (start 18.999998 41.999998) (end 19 42) (width 0.2) (layer "F.Cu") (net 9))
 (via (at 16 27.2) (size 0.6) (drill 0.3) (layers "F.Cu" "B.Cu") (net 9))
 (via (at 19 42) (size 0.6) (drill 0.3) (layers "F.Cu" "B.Cu") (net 9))
 (segment (start 16 39) (end 16 27.2) (width 0.2) (layer "B.Cu") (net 9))
 (segment (start 19 42) (end 16 39) (width 0.2) (layer "B.Cu") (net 9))
 (segment (start 33.0175 32.1825) (end 34.901 32.1825) (width 0.2) (layer "F.Cu") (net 7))
 (segment (start 27.99 56.42) (end 27.99 37.21) (width 0.2) (layer "F.Cu") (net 7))
 (segment (start 27.99 37.21) (end 33.0175 32.1825) (width 0.2) (layer "F.Cu") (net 7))
 (segment (start 26.589 37.1195) (end 34.066 29.6425) (width 0.2) (layer "F.Cu") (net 4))
 (segment (start 27.99 58.401314) (end 26.589 57.000314) (width 0.2) (layer "F.Cu") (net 4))
 (segment (start 26.589 57.000314) (end 26.589 37.1195) (width 0.2) (layer "F.Cu") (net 4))
 (segment (start 41.4 31.4) (end 40.2 30.2) (width 0.2) (layer "F.Cu") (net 4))
 (segment (start 27.99 75.47) (end 27.99 58.401314) (width 0.2) (layer "F.Cu") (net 4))
 (segment (start 58.35 31.4) (end 41.4 31.4) (width 0.2) (layer "F.Cu") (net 4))
 (segment (start 62.75 27) (end 58.35 31.4) (width 0.2) (layer "F.Cu") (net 4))
 (via (at 40.2 30.2) (size 0.6) (drill 0.3) (layers "F.Cu" "B.Cu") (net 4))
 (segment (start 39.6425 29.6425) (end 34.066 29.6425) (width 0.2) (layer "B.Cu") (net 4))
 (segment (start 40.2 30.2) (end 39.6425 29.6425) (width 0.2) (layer "B.Cu") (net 4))
 (segment (start 32 25.0365) (end 34.066 27.1025) (width 0.2) (layer "F.Cu") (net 11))
 (segment (start 73 15.8) (end 71.801 14.601) (width 0.2) (layer "F.Cu") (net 11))
 (segment (start 66.09 56.42) (end 73 49.51) (width 0.2) (layer "F.Cu") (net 11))
 (segment (start 32 14.601) (end 32 25.0365) (width 0.2) (layer "F.Cu") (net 11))
 (segment (start 73 49.51) (end 73 15.8) (width 0.2) (layer "F.Cu") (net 11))
 (segment (start 71.801 14.601) (end 32 14.601) (width 0.2) (layer "F.Cu") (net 11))
 (segment (start 38.2 66.63) (end 38.2 27.8615) (width 0.2) (layer "F.Cu") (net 12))
 (segment (start 47.04 75.47) (end 38.2 66.63) (width 0.2) (layer "F.Cu") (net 12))
 (segment (start 38.2 27.8615) (end 34.901 24.5625) (width 0.2) (layer "F.Cu") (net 12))
 (segment (start 40.730231 29.599) (end 40.774597 29.643366) (width 0.2) (layer "F.Cu") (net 8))
 (segment (start 48.430057 39.28) (end 39.599 30.448943) (width 0.2) (layer "F.Cu") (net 8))
 (segment (start 39.951057 29.599) (end 40.730231 29.599) (width 0.2) (layer "F.Cu") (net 8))
 (segment (start 39.599 29.951057) (end 39.951057 29.599) (width 0.2) (layer "F.Cu") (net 8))
 (segment (start 39.599 30.448943) (end 39.599 29.951057) (width 0.2) (layer "F.Cu") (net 8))
 (segment (start 66.4 39.28) (end 48.430057 39.28) (width 0.2) (layer "F.Cu") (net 8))
 (via (at 40.774597 29.643366) (size 0.6) (drill 0.3) (layers "F.Cu" "B.Cu") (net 8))
 (segment (start 19.26631 23.0855) (end 19.889 22.46281) (width 0.2) (layer "B.Cu") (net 8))
 (segment (start 26.5547 28.5795) (end 24.0277 31.1065) (width 0.2) (layer "B.Cu") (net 8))
 (segment (start 24.0277 31.1065) (end 18.21959 31.1065) (width 0.2) (layer "B.Cu") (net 8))
 (segment (start 18.21959 31.1065) (end 17.362 30.24891) (width 0.2) (layer "B.Cu") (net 8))
 (segment (start 17.362 30.24891) (end 17.362 24.52319) (width 0.2) (layer "B.Cu") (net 8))
 (segment (start 39.710731 28.5795) (end 26.5547 28.5795) (width 0.2) (layer "B.Cu") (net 8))
 (segment (start 40.774597 29.643366) (end 39.710731 28.5795) (width 0.2) (layer "B.Cu") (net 8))
 (segment (start 17.362 24.52319) (end 18.79969 23.0855) (width 0.2) (layer "B.Cu") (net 8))
 (segment (start 19.889 18.0055) (end 18.826 16.9425) (width 0.2) (layer "B.Cu") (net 8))
 (segment (start 19.889 22.46281) (end 19.889 18.0055) (width 0.2) (layer "B.Cu") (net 8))
 (segment (start 18.79969 23.0855) (end 19.26631 23.0855) (width 0.2) (layer "B.Cu") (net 8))
 (segment (start 35.14363 22.0225) (end 34.066 22.0225) (width 0.2) (layer "F.Cu") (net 13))
 (segment (start 38.601 27.547126) (end 36.418 25.364126) (width 0.2) (layer "F.Cu") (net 13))
 (segment (start 66.4 44.36) (end 50.36 44.36) (width 0.2) (layer "F.Cu") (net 13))
 (segment (start 36.418 25.364126) (end 36.418 23.29687) (width 0.2) (layer "F.Cu") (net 13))
 (segment (start 50.36 44.36) (end 38.601 32.601) (width 0.2) (layer "F.Cu") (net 13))
 (segment (start 38.601 32.601) (end 38.601 27.547126) (width 0.2) (layer "F.Cu") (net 13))
 (segment (start 36.418 23.29687) (end 35.14363 22.0225) (width 0.2) (layer "F.Cu") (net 13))
 (segment (start 14.601 87.801) (end 14.601 18.6) (width 0.2) (layer "F.Cu") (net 5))
 (segment (start 15.4835 19.4825) (end 18.826 19.4825) (width 0.2) (layer "F.Cu") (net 5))
 (segment (start 38.999 89.6) (end 16 89.6) (width 0.2) (layer "F.Cu") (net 5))
 (segment (start 48.441 74.889686) (end 48.441 80.158) (width 0.2) (layer "F.Cu") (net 5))
 (segment (start 16 89.6) (end 16 89.2) (width 0.2) (layer "F.Cu") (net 5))
 (segment (start 47.04 56.42) (end 47.04 73.488686) (width 0.2) (layer "F.Cu") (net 5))
 (segment (start 14.601 18.6) (end 15.4835 19.4825) (width 0.2) (layer "F.Cu") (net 5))
 (segment (start 48.441 80.158) (end 38.999 89.6) (width 0.2) (layer "F.Cu") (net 5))
 (segment (start 16 89.2) (end 14.601 87.801) (width 0.2) (layer "F.Cu") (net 5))
 (segment (start 47.04 73.488686) (end 48.441 74.889686) (width 0.2) (layer "F.Cu") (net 5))
 (segment (start 57.73 75.47) (end 43 90.2) (width 0.2) (layer "F.Cu") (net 6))
 (segment (start 66.09 75.47) (end 57.73 75.47) (width 0.2) (layer "F.Cu") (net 6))
 (via (at 43 90.2) (size 0.6) (drill 0.3) (layers "F.Cu" "B.Cu") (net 6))
 (segment (start 20 90.2) (end 14.601 84.801) (width 0.2) (layer "B.Cu") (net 6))
 (segment (start 14.601 84.801) (end 14.601 22) (width 0.2) (layer "B.Cu") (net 6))
 (segment (start 14.6235 22.0225) (end 18.826 22.0225) (width 0.2) (layer "B.Cu") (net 6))
 (segment (start 14.601 22) (end 14.6235 22.0225) (width 0.2) (layer "B.Cu") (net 6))
 (segment (start 43 90.2) (end 20 90.2) (width 0.2) (layer "B.Cu") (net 6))
 (segment (start 39.5005 23.4995) (end 38 25) (width 0.2) (layer "F.Cu") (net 2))
 (segment (start 44.7495 23.4995) (end 39.5005 23.4995) (width 0.2) (layer "F.Cu") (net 2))
 (segment (start 48.25 27) (end 44.7495 23.4995) (width 0.2) (layer "F.Cu") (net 2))
 (via (at 38 25) (size 0.6) (drill 0.3) (layers "F.Cu" "B.Cu") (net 2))
 (segment (start 18.38569 30.7055) (end 17.763 30.08281) (width 0.2) (layer "B.Cu") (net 2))
 (segment (start 31.0676 23.4995) (end 23.8616 30.7055) (width 0.2) (layer "B.Cu") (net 2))
 (segment (start 38 25) (end 36.4995 23.4995) (width 0.2) (layer "B.Cu") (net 2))
 (segment (start 23.8616 30.7055) (end 18.38569 30.7055) (width 0.2) (layer "B.Cu") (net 2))
 (segment (start 36.4995 23.4995) (end 31.0676 23.4995) (width 0.2) (layer "B.Cu") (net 2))
 (segment (start 17.763 30.08281) (end 17.763 25.6255) (width 0.2) (layer "B.Cu") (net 2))
 (segment (start 17.763 25.6255) (end 18.826 24.5625) (width 0.2) (layer "B.Cu") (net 2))
 (segment (start 48.25 22) (end 47.05 20.8) (width 0.2) (layer "F.Cu") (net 1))
 (segment (start 47.05 20.8) (end 46.6 20.8) (width 0.2) (layer "F.Cu") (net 1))
 (via (at 46.6 20.8) (size 0.6) (drill 0.3) (layers "F.Cu" "B.Cu") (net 1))
 (segment (start 24.3575 29.6425) (end 18.826 29.6425) (width 0.2) (layer "B.Cu") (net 1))
 (segment (start 33.2 20.8) (end 24.3575 29.6425) (width 0.2) (layer "B.Cu") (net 1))
 (segment (start 46.6 20.8) (end 33.2 20.8) (width 0.2) (layer "B.Cu") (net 1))
 (segment (start 24.773874 40.45) (end 25.6 41.276126) (width 0.2) (layer "F.Cu") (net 16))
 (segment (start 25 49) (end 20.078297 49) (width 0.2) (layer "F.Cu") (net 16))
 (segment (start 20.078297 49) (end 19.336039 48.257742) (width 0.2) (layer "F.Cu") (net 16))
 (segment (start 25.6 41.276126) (end 25.6 44) (width 0.2) (layer "F.Cu") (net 16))
 (segment (start 24.199998 40.45) (end 24.773874 40.45) (width 0.2) (layer "F.Cu") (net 16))
 (via (at 25.6 44) (size 0.6) (drill 0.3) (layers "F.Cu" "B.Cu") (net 16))
 (via (at 18.999998 47) (size 0.6) (drill 0.3) (layers "F.Cu" "B.Cu") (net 16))
 (via (at 19.336039 48.257742) (size 0.6) (drill 0.3) (layers "F.Cu" "B.Cu") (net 16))
 (via (at 25 49) (size 0.6) (drill 0.3) (layers "F.Cu" "B.Cu") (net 16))
 (segment (start 27 45.4) (end 25.6 44) (width 0.2) (layer "B.Cu") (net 16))
 (segment (start 26.2 48.4) (end 25.6 48.4) (width 0.2) (layer "B.Cu") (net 16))
 (segment (start 19.336039 48.257742) (end 18.999998 47.921701) (width 0.2) (layer "B.Cu") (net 16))
 (segment (start 27 47.6) (end 26.2 48.4) (width 0.2) (layer "B.Cu") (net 16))
 (segment (start 27 47.6) (end 27 45.4) (width 0.2) (layer "B.Cu") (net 16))
 (segment (start 18.999998 47.921701) (end 18.999998 47) (width 0.2) (layer "B.Cu") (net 16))
 (segment (start 25.6 48.4) (end 25 49) (width 0.2) (layer "B.Cu") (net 16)))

